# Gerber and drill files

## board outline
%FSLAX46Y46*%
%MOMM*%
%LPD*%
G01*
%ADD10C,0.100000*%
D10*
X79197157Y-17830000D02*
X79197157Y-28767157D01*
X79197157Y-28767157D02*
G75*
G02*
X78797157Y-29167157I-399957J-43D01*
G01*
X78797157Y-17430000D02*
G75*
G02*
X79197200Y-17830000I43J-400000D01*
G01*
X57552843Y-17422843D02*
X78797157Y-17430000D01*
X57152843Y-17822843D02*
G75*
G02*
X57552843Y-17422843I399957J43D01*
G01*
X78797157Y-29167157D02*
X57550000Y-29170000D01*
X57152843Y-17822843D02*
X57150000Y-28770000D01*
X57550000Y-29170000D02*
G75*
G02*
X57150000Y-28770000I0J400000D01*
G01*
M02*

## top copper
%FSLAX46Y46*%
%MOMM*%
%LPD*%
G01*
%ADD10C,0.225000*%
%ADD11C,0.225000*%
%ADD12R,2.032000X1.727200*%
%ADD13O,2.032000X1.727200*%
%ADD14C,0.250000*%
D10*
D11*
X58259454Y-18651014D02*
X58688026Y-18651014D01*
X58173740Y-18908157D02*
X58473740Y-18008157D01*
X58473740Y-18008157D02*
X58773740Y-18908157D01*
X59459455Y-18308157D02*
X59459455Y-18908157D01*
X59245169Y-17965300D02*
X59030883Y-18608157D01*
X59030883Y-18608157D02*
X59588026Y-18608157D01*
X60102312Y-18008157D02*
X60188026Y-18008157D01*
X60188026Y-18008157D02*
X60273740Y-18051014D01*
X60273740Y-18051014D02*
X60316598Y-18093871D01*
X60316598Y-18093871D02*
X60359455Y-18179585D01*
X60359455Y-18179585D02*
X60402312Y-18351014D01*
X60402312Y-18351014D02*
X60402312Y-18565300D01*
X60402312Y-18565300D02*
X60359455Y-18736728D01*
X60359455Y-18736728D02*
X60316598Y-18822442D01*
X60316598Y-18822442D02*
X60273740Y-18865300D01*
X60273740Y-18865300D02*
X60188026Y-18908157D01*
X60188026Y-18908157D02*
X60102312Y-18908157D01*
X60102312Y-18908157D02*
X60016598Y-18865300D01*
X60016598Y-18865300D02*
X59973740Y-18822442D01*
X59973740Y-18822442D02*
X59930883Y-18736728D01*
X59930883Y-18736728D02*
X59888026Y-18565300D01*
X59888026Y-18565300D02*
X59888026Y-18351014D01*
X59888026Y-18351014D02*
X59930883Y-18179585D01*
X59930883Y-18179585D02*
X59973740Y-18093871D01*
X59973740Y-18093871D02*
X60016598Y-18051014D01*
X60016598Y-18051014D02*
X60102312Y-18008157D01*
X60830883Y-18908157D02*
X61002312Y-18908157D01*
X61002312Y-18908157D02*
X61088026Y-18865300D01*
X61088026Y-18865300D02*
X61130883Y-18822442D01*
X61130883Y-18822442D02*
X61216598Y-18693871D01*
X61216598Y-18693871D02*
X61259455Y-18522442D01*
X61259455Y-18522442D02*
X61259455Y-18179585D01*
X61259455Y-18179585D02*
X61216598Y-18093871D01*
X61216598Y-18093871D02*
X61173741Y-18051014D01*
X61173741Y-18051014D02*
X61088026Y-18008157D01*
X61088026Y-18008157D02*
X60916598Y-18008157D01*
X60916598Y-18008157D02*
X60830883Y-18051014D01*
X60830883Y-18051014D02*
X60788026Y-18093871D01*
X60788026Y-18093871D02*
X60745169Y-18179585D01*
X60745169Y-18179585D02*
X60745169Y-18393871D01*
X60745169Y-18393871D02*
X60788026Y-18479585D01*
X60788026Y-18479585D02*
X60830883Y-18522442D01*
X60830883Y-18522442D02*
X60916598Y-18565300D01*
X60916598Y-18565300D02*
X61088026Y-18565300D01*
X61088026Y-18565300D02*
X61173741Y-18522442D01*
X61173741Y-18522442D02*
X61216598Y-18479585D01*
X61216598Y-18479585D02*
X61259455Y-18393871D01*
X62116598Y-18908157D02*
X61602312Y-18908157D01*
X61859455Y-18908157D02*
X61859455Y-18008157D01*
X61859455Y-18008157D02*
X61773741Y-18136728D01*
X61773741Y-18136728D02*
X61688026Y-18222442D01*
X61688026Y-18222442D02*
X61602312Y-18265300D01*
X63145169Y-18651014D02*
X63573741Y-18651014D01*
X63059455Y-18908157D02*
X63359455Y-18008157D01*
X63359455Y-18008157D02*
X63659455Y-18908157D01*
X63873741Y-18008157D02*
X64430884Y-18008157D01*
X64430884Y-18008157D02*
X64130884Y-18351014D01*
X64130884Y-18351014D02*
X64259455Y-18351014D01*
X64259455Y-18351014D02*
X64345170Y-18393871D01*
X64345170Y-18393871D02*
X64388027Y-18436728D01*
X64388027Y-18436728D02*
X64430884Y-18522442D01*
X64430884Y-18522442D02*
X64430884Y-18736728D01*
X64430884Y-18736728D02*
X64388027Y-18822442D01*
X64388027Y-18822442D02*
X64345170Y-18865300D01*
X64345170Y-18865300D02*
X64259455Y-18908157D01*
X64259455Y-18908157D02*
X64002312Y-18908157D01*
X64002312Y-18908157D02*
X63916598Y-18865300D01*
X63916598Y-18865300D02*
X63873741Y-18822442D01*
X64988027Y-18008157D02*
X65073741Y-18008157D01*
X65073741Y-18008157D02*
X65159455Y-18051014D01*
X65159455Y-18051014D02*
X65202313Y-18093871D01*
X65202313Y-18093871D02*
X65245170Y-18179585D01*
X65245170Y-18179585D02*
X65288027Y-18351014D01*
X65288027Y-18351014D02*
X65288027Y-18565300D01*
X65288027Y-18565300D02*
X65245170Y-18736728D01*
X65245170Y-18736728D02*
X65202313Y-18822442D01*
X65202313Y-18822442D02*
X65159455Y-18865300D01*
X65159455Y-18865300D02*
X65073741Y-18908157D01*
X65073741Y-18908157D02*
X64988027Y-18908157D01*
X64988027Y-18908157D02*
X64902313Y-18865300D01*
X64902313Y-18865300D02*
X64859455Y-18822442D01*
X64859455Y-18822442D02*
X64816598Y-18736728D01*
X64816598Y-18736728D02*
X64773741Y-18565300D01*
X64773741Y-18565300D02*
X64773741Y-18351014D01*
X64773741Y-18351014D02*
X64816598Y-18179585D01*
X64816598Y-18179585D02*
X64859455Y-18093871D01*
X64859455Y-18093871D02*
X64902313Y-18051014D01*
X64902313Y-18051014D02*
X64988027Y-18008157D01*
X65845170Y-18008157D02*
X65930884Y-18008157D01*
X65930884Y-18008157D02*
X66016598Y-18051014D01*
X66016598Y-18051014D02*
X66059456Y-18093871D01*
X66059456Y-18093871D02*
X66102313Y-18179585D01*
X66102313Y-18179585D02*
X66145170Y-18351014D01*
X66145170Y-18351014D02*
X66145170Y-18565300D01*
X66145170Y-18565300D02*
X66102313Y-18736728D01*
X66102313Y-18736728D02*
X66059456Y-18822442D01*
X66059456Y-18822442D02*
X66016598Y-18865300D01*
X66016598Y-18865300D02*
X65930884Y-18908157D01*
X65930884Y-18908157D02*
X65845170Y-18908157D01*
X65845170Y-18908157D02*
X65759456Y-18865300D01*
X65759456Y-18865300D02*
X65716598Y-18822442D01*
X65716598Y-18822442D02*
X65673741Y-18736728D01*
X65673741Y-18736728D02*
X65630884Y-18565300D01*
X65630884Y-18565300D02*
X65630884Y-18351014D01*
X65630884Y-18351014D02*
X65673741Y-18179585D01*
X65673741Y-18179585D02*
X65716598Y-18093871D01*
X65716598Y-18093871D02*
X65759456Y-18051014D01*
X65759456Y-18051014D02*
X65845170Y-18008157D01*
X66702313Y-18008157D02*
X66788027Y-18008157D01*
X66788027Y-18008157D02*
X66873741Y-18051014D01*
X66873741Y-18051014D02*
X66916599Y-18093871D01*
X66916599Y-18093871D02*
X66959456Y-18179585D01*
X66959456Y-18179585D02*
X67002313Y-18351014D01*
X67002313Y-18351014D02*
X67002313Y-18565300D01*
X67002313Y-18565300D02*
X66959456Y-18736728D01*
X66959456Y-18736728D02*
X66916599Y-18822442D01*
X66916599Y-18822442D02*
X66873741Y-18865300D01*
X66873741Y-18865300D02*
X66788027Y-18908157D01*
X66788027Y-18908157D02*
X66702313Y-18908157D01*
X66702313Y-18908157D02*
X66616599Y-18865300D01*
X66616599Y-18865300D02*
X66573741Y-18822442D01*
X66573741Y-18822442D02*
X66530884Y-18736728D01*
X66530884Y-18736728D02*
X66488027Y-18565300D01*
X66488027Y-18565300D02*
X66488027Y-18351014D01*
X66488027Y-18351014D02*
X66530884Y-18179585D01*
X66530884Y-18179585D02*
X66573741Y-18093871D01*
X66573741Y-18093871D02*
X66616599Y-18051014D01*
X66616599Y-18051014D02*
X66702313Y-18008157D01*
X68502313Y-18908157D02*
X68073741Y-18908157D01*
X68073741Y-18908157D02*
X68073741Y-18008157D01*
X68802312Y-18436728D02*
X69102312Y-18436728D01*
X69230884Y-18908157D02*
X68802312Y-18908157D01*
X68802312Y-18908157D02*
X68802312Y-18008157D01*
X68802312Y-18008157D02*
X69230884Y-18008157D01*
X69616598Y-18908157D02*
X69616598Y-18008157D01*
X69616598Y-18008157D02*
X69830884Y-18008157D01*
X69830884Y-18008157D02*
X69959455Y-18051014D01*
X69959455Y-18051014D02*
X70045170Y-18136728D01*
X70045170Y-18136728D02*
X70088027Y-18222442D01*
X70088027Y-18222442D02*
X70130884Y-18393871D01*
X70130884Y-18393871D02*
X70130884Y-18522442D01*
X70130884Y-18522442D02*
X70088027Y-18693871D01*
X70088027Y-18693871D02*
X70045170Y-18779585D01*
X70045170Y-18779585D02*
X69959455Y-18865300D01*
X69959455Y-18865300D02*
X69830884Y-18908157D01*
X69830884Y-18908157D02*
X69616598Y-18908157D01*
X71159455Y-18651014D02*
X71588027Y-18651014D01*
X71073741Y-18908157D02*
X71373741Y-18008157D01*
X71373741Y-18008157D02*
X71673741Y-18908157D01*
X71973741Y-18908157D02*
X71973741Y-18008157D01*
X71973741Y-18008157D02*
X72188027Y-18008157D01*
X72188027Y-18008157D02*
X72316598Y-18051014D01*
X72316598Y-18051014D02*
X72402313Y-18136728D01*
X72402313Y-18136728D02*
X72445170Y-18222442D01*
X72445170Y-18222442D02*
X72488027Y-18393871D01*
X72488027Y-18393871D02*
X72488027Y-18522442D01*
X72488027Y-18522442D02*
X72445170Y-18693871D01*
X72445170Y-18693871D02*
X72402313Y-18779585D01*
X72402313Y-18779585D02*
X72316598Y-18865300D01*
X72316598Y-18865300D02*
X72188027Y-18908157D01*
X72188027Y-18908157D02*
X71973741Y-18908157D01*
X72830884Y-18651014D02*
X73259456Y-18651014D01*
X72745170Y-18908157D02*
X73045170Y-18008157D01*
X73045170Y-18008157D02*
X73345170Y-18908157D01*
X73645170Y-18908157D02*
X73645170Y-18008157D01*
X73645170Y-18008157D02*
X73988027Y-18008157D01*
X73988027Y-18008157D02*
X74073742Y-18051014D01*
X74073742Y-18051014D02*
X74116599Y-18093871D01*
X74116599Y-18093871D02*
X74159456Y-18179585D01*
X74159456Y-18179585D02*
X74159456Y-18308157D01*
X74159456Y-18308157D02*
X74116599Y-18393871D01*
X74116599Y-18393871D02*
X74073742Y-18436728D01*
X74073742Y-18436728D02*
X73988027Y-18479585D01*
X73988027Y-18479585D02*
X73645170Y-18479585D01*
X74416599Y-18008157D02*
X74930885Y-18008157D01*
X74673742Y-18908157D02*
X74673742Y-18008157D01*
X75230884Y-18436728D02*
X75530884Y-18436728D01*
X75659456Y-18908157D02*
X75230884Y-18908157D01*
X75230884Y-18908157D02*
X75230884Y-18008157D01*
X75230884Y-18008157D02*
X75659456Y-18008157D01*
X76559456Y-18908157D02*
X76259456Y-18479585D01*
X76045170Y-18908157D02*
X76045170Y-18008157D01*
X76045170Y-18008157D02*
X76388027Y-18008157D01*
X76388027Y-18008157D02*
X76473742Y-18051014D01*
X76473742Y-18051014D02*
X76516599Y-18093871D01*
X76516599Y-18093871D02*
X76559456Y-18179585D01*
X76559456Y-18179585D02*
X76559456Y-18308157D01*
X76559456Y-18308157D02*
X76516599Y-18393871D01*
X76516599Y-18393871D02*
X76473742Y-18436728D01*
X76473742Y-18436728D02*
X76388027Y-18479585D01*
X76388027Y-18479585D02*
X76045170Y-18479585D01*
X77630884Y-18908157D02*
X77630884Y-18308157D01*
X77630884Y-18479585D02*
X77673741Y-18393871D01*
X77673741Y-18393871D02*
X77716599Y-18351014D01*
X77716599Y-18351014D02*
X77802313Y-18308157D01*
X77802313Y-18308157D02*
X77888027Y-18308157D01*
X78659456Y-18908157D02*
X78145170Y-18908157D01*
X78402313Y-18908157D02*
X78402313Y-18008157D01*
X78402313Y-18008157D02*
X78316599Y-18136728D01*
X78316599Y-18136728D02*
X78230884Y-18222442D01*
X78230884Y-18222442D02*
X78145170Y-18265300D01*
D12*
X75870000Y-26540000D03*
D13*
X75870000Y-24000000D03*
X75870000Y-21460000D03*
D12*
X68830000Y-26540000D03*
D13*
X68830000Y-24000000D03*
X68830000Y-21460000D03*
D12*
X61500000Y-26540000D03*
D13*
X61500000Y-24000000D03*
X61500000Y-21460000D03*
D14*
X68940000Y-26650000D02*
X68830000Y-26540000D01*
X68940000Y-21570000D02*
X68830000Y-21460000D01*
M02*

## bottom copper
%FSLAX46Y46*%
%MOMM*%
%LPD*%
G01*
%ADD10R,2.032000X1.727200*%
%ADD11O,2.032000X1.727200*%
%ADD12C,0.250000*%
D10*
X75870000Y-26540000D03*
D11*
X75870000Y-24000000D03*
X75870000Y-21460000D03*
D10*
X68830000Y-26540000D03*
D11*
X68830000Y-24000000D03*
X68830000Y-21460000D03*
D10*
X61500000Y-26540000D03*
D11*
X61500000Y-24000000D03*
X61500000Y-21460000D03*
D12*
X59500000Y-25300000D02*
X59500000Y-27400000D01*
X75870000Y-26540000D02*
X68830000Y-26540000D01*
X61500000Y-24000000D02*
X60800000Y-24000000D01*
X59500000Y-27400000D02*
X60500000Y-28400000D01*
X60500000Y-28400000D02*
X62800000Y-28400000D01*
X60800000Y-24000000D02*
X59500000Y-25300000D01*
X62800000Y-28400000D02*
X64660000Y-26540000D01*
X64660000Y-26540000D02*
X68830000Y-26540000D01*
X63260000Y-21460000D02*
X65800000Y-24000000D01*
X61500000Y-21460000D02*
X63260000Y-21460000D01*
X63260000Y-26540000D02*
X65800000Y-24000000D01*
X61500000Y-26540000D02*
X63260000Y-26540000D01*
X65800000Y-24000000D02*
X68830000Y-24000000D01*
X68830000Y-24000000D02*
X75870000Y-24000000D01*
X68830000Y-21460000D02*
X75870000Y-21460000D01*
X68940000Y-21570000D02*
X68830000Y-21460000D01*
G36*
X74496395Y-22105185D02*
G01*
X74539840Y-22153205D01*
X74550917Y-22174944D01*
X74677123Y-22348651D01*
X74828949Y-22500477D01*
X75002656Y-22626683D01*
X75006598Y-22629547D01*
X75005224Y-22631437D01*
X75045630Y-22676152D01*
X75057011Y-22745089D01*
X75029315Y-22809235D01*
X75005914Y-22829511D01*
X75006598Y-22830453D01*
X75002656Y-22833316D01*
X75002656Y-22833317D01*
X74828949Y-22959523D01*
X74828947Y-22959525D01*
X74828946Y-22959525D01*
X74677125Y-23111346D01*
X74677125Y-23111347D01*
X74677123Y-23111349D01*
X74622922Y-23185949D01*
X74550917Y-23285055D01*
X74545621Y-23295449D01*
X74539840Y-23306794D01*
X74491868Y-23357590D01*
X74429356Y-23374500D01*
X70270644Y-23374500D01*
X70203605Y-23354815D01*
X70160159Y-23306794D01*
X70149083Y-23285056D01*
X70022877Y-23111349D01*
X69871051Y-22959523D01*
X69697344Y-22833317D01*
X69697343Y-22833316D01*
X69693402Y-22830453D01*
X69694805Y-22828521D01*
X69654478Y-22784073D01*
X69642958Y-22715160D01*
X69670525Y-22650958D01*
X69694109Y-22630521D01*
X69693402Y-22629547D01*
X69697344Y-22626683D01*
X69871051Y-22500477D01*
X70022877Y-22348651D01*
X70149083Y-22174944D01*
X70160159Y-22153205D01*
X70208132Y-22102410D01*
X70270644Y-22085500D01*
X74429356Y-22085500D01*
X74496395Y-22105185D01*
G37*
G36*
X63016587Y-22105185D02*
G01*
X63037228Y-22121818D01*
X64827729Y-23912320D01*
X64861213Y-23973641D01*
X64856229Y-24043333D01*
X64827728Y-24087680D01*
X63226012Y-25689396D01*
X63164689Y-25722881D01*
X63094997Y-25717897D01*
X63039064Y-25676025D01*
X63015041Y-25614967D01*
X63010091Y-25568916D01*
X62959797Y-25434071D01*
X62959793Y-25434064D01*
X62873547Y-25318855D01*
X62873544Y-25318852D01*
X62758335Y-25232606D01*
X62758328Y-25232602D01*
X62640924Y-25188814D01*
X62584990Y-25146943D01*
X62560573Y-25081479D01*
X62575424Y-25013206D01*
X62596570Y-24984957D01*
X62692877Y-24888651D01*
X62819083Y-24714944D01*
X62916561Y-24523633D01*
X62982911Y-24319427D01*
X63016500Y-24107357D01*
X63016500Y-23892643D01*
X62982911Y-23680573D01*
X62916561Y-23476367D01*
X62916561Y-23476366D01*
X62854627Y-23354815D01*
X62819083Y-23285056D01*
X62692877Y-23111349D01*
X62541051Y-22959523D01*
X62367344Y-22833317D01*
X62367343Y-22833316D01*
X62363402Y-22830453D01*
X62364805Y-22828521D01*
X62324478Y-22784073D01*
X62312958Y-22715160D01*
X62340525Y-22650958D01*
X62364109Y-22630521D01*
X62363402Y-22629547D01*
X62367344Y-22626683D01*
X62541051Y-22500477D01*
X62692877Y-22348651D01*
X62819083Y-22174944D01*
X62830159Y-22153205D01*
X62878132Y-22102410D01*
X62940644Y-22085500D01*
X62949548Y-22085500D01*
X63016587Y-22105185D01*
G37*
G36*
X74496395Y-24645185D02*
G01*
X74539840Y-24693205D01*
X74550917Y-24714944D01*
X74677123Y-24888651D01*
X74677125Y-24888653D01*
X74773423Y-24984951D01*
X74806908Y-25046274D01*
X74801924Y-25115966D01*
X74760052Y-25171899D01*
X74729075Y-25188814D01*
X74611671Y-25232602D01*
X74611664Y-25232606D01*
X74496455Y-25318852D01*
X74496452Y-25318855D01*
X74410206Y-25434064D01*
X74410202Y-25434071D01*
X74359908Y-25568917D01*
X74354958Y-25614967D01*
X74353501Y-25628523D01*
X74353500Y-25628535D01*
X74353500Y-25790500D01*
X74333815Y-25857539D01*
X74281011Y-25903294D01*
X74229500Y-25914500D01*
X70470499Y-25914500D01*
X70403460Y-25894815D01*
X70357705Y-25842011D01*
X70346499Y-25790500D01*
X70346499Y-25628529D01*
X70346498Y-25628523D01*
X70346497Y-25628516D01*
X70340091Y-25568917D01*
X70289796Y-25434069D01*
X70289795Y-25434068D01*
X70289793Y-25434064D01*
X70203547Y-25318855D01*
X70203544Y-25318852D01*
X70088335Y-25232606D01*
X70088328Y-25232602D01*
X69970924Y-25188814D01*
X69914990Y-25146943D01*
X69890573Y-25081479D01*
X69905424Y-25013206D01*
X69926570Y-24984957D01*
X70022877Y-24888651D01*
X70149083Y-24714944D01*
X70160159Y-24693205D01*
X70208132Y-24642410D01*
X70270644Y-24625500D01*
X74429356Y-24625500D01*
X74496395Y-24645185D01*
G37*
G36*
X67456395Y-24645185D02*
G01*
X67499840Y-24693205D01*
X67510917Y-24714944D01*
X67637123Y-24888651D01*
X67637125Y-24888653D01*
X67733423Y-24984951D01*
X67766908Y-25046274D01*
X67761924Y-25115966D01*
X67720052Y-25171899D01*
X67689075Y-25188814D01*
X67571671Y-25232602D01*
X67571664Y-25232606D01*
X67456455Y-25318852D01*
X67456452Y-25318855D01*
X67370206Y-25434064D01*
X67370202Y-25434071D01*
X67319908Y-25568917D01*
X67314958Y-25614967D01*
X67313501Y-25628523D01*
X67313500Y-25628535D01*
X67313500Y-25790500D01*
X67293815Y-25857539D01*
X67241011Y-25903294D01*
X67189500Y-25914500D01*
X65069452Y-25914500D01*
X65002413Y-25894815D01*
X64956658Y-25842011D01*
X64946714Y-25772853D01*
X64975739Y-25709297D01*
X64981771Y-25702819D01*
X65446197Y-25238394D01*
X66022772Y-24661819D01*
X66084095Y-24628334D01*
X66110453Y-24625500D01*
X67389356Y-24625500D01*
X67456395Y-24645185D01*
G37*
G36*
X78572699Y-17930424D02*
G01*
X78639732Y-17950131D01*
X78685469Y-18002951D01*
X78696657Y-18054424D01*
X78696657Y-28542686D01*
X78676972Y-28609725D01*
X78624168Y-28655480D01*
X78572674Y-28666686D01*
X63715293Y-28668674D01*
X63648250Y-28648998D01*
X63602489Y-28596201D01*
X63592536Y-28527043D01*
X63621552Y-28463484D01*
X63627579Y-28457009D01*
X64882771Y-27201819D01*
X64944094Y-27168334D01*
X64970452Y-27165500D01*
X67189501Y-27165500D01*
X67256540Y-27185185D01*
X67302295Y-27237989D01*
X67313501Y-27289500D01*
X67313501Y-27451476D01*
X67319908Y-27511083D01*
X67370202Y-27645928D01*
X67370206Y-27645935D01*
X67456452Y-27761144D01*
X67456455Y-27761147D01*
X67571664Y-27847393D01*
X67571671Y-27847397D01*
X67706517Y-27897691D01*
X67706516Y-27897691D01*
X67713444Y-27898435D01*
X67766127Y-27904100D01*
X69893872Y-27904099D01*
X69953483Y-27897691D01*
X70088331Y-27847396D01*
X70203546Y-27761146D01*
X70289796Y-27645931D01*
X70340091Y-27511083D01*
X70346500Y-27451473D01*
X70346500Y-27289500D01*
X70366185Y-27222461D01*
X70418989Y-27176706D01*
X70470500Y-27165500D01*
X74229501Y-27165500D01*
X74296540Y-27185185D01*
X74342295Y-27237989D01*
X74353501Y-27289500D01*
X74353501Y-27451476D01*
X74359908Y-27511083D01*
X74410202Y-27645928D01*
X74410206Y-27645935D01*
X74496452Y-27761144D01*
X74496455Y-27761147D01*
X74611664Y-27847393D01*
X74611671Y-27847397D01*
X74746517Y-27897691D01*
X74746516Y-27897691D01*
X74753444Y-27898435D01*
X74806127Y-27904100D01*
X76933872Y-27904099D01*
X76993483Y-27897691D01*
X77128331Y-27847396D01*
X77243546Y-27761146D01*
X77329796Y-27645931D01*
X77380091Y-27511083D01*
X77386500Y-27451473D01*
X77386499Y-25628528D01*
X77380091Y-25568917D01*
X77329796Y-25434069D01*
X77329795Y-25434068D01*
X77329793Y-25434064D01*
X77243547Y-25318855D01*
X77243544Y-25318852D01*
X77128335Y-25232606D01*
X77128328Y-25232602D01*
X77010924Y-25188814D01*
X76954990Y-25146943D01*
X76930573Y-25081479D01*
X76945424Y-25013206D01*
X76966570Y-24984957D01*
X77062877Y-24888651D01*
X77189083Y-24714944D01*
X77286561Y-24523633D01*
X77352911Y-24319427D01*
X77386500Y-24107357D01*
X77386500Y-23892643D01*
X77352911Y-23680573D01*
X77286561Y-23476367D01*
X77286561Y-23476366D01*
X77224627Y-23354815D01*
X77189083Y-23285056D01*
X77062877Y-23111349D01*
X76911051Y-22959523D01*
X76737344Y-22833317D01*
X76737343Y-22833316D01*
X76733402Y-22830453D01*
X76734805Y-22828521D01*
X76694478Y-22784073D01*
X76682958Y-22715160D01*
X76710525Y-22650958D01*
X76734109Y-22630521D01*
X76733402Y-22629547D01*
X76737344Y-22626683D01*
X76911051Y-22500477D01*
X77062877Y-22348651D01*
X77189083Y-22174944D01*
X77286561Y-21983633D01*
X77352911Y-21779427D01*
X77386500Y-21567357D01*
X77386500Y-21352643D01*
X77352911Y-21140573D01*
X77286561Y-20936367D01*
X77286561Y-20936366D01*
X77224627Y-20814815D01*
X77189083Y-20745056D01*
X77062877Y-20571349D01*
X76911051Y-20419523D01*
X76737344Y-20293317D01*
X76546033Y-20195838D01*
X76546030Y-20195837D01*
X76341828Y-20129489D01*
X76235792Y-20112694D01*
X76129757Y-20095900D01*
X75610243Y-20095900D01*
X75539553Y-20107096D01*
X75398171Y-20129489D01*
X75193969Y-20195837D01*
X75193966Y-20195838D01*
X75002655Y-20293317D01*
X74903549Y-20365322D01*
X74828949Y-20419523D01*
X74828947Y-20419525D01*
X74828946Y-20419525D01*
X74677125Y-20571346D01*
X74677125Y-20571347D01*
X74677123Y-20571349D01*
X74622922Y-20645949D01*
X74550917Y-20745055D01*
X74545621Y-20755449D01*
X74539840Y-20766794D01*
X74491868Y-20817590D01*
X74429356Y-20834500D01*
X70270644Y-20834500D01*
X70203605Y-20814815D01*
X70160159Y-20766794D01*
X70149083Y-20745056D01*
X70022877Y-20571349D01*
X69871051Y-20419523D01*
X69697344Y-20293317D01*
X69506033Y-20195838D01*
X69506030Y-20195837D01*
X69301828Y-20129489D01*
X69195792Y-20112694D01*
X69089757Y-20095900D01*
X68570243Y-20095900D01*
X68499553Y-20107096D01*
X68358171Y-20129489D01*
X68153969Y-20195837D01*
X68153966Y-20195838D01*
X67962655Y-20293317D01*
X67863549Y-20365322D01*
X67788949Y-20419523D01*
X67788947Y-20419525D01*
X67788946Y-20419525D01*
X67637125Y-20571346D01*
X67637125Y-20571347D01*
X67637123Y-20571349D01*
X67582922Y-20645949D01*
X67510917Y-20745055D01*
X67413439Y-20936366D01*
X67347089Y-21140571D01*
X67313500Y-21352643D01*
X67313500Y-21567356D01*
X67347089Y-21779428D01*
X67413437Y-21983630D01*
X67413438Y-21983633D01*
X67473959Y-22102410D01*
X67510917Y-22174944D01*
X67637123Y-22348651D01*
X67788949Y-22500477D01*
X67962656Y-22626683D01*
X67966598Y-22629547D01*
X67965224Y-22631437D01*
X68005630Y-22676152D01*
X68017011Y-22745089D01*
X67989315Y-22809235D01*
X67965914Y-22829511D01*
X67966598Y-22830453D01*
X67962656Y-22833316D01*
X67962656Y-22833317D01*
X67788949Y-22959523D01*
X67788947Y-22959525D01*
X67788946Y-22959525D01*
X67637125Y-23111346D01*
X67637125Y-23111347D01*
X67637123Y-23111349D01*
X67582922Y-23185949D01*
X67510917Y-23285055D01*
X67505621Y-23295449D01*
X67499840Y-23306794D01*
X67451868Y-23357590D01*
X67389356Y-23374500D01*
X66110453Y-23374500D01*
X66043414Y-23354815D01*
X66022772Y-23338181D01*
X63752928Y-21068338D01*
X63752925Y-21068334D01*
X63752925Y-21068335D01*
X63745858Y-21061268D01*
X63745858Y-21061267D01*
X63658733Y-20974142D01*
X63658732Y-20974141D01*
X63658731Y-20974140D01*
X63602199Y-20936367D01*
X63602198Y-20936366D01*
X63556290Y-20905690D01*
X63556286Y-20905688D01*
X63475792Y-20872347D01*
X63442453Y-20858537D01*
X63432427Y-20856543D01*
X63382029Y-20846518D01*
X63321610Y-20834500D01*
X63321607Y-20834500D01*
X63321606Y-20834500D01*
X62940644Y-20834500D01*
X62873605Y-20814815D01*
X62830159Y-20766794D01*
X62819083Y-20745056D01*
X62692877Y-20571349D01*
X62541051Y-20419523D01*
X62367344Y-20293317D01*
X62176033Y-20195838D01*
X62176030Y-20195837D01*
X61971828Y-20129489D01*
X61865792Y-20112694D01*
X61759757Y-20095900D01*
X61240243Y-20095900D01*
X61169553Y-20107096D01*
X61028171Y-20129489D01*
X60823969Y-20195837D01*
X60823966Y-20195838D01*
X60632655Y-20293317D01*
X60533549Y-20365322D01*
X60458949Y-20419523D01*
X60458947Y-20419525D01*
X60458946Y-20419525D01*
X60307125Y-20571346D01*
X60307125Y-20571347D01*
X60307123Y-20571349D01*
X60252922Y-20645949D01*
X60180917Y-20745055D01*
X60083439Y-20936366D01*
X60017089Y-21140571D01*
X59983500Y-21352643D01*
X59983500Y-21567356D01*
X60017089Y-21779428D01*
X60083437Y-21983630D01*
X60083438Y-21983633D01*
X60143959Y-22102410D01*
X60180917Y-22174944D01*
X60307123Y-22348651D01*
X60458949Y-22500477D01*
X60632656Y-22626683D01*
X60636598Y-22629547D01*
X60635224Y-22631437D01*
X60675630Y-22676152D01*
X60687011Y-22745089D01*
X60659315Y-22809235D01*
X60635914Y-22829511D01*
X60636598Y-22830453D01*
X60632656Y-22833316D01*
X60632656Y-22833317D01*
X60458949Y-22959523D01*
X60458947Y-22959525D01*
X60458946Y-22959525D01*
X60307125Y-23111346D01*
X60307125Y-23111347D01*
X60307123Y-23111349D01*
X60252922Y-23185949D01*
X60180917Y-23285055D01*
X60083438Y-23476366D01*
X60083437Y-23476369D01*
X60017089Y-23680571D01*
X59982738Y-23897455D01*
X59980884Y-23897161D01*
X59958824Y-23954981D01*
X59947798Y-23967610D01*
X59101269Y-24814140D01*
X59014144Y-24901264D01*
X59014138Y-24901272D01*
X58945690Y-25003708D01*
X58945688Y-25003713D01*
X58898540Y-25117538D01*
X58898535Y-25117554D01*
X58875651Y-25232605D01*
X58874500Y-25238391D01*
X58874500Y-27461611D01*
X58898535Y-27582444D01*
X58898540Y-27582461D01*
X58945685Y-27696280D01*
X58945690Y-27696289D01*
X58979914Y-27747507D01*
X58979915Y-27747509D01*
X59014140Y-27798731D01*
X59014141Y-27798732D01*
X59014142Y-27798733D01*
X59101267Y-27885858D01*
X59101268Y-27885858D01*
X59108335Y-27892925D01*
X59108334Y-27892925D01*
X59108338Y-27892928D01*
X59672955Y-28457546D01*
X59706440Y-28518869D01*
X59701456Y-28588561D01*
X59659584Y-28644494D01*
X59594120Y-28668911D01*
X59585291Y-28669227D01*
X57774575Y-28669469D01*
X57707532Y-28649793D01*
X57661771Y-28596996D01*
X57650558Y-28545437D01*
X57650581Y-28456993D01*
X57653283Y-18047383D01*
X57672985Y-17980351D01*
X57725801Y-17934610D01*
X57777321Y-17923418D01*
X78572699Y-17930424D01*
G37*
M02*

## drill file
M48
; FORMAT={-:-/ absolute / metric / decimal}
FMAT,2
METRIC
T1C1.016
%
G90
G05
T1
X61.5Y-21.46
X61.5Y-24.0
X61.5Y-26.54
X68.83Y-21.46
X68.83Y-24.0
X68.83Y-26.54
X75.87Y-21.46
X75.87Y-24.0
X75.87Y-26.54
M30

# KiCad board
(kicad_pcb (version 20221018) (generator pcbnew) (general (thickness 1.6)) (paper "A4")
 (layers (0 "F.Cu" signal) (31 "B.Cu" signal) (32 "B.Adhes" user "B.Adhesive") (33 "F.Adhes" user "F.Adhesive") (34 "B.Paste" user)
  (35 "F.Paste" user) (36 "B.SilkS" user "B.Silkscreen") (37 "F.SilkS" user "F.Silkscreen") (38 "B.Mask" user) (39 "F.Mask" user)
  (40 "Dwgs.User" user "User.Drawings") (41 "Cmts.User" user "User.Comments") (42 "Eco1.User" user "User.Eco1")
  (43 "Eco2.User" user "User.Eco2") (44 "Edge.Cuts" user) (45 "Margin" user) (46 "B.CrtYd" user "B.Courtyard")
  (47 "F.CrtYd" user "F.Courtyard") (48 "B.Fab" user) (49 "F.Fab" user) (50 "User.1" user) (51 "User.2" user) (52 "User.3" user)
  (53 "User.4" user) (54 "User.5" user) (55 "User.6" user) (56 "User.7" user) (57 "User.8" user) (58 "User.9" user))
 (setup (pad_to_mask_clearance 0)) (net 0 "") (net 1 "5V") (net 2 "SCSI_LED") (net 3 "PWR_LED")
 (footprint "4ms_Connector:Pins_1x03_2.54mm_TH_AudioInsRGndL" (layer "F.Cu") (at 75.87 24 180)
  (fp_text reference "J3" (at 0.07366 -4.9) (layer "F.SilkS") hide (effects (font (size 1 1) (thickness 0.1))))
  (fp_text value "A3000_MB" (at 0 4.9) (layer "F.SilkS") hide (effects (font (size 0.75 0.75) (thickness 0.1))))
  (pad "1" thru_hole rect (at 0 -2.54 180) (size 2.032 1.7272) (drill 1.016) (layers "*.Cu" "*.Mask") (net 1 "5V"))
  (pad "2" thru_hole oval (at 0 0 180) (size 2.032 1.7272) (drill 1.016) (layers "*.Cu" "*.Mask") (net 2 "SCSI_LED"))
  (pad "3" thru_hole oval (at 0 2.54 180) (size 2.032 1.7272) (drill 1.016) (layers "*.Cu" "*.Mask") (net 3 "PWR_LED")))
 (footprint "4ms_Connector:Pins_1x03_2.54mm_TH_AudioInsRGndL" (layer "F.Cu") (at 68.83 24 180)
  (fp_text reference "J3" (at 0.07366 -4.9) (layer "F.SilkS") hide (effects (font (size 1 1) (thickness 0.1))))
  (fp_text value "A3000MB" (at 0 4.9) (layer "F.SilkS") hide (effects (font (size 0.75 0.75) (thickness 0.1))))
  (pad "1" thru_hole rect (at 0 -2.54 180) (size 2.032 1.7272) (drill 1.016) (layers "*.Cu" "*.Mask") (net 1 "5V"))
  (pad "2" thru_hole oval (at 0 0 180) (size 2.032 1.7272) (drill 1.016) (layers "*.Cu" "*.Mask") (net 2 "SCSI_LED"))
  (pad "3" thru_hole oval (at 0 2.54 180) (size 2.032 1.7272) (drill 1.016) (layers "*.Cu" "*.Mask") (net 3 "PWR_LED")))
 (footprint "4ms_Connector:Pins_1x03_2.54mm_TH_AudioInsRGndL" (layer "F.Cu") (at 61.5 24 180)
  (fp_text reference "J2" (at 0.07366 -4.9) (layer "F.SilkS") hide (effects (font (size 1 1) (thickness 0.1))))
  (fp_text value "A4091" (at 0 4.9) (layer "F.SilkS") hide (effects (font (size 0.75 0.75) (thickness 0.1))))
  (pad "1" thru_hole rect (at 0 -2.54 180) (size 2.032 1.7272) (drill 1.016) (layers "*.Cu" "*.Mask") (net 2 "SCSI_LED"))
  (pad "2" thru_hole oval (at 0 0 180) (size 2.032 1.7272) (drill 1.016) (layers "*.Cu" "*.Mask") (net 1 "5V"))
  (pad "3" thru_hole oval (at 0 2.54 180) (size 2.032 1.7272) (drill 1.016) (layers "*.Cu" "*.Mask") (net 2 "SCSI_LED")))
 (gr_line (start 79.197157 17.83) (end 79.197157 28.767157) (stroke (width 0.1) (type default)) (layer "Edge.Cuts"))
 (gr_arc (start 79.197157 28.767157) (mid 79.08 29.05) (end 78.797157 29.167157) (stroke (width 0.1) (type default)) (layer "Edge.Cuts"))
 (gr_arc (start 78.797157 17.43) (mid 79.08 17.547157) (end 79.197157 17.83) (stroke (width 0.1) (type default)) (layer "Edge.Cuts"))
 (gr_line (start 57.552843 17.422843) (end 78.797157 17.43) (stroke (width 0.1) (type default)) (layer "Edge.Cuts"))
 (gr_arc (start 57.152843 17.822843) (mid 57.27 17.54) (end 57.552843 17.422843) (stroke (width 0.1) (type default)) (layer "Edge.Cuts"))
 (gr_line (start 78.797157 29.167157) (end 57.55 29.17) (stroke (width 0.1) (type default)) (layer "Edge.Cuts"))
 (gr_line (start 57.152843 17.822843) (end 57.15 28.77) (stroke (width 0.1) (type default)) (layer "Edge.Cuts"))
 (gr_arc (start 57.55 29.17) (mid 57.267157 29.052843) (end 57.15 28.77) (stroke (width 0.1) (type default)) (layer "Edge.Cuts"))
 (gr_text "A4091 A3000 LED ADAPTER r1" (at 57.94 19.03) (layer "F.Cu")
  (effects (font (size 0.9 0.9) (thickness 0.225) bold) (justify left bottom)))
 (segment (start 68.94 26.65) (end 68.83 26.54) (width 0.25) (layer "F.Cu") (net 1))
 (segment (start 59.5 25.3) (end 59.5 27.4) (width 0.25) (layer "B.Cu") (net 1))
 (segment (start 75.87 26.54) (end 68.83 26.54) (width 0.25) (layer "B.Cu") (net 1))
 (segment (start 61.5 24) (end 60.8 24) (width 0.25) (layer "B.Cu") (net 1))
 (segment (start 59.5 27.4) (end 60.5 28.4) (width 0.25) (layer "B.Cu") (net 1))
 (segment (start 60.5 28.4) (end 62.8 28.4) (width 0.25) (layer "B.Cu") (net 1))
 (segment (start 60.8 24) (end 59.5 25.3) (width 0.25) (layer "B.Cu") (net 1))
 (segment (start 62.8 28.4) (end 64.66 26.54) (width 0.25) (layer "B.Cu") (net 1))
 (segment (start 64.66 26.54) (end 68.83 26.54) (width 0.25) (layer "B.Cu") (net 1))
 (segment (start 63.26 21.46) (end 65.8 24) (width 0.25) (layer "B.Cu") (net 2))
 (segment (start 61.5 21.46) (end 63.26 21.46) (width 0.25) (layer "B.Cu") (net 2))
 (segment (start 63.26 26.54) (end 65.8 24) (width 0.25) (layer "B.Cu") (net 2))
 (segment (start 61.5 26.54) (end 63.26 26.54) (width 0.25) (layer "B.Cu") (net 2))
 (segment (start 65.8 24) (end 68.83 24) (width 0.25) (layer "B.Cu") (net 2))
 (segment (start 68.83 24) (end 75.87 24) (width 0.25) (layer "B.Cu") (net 2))
 (segment (start 68.94 21.57) (end 68.83 21.46) (width 0.25) (layer "F.Cu") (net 3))
 (segment (start 68.83 21.46) (end 75.87 21.46) (width 0.25) (layer "B.Cu") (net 3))
 (segment (start 68.94 21.57) (end 68.83 21.46) (width 0.25) (layer "B.Cu") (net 3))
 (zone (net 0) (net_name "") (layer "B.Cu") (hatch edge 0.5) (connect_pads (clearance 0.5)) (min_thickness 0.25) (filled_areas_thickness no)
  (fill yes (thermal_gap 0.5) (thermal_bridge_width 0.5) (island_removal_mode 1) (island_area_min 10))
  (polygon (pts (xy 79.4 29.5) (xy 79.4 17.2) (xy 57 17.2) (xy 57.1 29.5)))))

